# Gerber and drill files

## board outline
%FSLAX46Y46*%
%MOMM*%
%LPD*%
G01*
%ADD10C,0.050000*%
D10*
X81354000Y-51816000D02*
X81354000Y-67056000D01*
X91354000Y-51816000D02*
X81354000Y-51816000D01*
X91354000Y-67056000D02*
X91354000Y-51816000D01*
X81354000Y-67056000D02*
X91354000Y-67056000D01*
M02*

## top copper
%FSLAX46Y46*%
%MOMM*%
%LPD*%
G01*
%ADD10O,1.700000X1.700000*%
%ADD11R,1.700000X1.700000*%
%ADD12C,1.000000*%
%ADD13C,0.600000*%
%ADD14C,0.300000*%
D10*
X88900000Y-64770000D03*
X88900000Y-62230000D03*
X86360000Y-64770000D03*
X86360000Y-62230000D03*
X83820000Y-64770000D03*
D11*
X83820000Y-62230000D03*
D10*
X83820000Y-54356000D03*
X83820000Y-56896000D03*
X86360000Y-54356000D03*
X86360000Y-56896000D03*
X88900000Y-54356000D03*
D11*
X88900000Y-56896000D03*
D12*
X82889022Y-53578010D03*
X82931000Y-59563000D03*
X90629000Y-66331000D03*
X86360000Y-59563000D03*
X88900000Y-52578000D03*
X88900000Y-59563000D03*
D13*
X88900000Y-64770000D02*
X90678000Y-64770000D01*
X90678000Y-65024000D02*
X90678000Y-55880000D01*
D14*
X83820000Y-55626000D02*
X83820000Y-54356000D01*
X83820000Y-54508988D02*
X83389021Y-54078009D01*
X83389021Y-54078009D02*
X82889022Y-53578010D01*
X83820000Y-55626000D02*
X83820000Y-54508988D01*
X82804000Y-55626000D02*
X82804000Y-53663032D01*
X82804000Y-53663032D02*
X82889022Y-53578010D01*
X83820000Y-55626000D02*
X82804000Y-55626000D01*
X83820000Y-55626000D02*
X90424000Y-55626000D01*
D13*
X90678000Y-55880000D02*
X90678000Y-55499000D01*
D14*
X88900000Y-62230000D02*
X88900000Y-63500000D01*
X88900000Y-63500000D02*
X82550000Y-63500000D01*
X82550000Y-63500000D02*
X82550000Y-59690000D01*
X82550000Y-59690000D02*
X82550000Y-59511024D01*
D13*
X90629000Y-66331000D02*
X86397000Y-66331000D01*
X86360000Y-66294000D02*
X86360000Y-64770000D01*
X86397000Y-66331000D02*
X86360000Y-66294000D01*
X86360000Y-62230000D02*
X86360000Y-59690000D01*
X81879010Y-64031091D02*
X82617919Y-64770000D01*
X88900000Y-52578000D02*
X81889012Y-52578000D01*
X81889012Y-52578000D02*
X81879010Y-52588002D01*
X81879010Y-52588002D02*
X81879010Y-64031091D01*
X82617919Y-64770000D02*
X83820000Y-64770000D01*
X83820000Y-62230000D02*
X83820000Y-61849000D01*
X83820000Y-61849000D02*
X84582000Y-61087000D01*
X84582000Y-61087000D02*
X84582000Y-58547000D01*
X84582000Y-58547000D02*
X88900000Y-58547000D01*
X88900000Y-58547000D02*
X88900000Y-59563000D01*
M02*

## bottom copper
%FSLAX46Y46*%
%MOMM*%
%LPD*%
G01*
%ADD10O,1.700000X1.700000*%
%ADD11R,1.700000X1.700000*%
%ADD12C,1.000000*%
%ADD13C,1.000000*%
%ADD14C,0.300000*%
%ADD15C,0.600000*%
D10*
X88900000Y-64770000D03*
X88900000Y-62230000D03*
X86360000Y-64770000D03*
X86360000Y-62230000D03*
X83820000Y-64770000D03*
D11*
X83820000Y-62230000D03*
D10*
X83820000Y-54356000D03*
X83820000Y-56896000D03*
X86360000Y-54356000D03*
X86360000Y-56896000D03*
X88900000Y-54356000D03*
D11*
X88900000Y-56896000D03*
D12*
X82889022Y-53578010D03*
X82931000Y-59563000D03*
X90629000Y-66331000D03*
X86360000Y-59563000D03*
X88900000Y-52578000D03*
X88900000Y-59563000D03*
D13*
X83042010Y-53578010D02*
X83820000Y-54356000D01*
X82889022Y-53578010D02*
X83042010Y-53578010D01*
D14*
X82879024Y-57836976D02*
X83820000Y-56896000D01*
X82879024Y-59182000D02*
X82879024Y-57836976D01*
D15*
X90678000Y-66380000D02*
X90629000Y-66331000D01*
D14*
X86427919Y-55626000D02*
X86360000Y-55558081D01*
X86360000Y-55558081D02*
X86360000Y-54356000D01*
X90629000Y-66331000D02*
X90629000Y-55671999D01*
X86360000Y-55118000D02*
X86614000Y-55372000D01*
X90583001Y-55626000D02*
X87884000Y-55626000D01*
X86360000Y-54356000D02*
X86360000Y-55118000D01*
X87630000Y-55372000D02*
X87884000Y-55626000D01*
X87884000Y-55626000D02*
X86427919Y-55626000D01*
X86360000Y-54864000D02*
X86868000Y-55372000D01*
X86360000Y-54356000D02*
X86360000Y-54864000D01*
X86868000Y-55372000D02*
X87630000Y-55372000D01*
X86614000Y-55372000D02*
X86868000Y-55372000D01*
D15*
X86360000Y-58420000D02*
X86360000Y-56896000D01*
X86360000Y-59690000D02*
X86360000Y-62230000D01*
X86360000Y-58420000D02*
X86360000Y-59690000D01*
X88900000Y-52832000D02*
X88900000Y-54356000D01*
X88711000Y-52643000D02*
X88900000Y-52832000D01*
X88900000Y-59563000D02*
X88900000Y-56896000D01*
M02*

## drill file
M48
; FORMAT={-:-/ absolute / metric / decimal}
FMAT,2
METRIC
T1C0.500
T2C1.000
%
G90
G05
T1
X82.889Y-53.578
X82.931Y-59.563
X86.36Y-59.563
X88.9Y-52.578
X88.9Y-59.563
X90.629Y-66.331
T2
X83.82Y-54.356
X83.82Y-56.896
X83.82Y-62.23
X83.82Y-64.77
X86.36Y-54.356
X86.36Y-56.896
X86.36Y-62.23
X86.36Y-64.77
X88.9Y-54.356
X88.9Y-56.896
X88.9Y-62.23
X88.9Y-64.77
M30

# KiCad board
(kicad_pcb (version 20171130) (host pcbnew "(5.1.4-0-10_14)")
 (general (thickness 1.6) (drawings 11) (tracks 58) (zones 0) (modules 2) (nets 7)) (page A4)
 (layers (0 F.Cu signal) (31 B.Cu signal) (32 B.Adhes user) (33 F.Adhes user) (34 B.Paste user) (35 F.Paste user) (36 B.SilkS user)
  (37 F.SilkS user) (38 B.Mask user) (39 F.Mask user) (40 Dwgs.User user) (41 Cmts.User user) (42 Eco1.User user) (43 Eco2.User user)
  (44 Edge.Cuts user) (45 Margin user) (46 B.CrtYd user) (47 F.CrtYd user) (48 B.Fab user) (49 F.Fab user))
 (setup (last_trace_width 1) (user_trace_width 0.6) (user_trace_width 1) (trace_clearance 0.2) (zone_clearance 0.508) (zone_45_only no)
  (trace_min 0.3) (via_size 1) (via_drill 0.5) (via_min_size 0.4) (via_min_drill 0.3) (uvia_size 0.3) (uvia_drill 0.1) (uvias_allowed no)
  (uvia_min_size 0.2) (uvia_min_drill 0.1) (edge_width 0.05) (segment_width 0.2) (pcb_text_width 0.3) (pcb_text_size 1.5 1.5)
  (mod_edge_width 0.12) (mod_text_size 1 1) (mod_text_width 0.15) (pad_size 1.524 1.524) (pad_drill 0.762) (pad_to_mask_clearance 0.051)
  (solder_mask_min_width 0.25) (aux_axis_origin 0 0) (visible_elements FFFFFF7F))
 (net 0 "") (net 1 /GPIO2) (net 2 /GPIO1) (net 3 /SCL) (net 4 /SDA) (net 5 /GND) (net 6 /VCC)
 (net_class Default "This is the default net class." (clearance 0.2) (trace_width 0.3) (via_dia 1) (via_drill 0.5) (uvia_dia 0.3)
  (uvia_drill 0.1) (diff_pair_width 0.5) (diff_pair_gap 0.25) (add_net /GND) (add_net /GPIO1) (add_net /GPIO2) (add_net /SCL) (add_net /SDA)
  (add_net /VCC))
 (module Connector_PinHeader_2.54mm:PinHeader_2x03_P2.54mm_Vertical (layer B.Cu) (at 83.82 62.23 270)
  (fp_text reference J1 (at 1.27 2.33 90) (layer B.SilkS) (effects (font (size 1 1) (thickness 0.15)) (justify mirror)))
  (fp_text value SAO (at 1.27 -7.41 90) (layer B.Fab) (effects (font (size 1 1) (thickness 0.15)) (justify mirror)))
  (pad 6 thru_hole oval (at 2.54 -5.08 270) (size 1.7 1.7) (drill 1) (layers *.Cu *.Mask) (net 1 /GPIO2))
  (pad 5 thru_hole oval (at 0 -5.08 270) (size 1.7 1.7) (drill 1) (layers *.Cu *.Mask) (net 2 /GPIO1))
  (pad 4 thru_hole oval (at 2.54 -2.54 270) (size 1.7 1.7) (drill 1) (layers *.Cu *.Mask) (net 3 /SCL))
  (pad 3 thru_hole oval (at 0 -2.54 270) (size 1.7 1.7) (drill 1) (layers *.Cu *.Mask) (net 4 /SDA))
  (pad 2 thru_hole oval (at 2.54 0 270) (size 1.7 1.7) (drill 1) (layers *.Cu *.Mask) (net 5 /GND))
  (pad 1 thru_hole rect (at 0 0 270) (size 1.7 1.7) (drill 1) (layers *.Cu *.Mask) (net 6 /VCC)))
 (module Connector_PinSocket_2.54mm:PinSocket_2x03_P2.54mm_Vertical (layer F.Cu) (at 88.9 56.896 270)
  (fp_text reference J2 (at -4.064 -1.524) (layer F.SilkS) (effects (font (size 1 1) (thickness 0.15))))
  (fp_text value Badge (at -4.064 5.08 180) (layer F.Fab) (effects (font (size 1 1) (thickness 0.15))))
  (pad 6 thru_hole oval (at -2.54 5.08 270) (size 1.7 1.7) (drill 1) (layers *.Cu *.Mask) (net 1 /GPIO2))
  (pad 5 thru_hole oval (at 0 5.08 270) (size 1.7 1.7) (drill 1) (layers *.Cu *.Mask) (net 2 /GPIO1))
  (pad 4 thru_hole oval (at -2.54 2.54 270) (size 1.7 1.7) (drill 1) (layers *.Cu *.Mask) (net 3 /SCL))
  (pad 3 thru_hole oval (at 0 2.54 270) (size 1.7 1.7) (drill 1) (layers *.Cu *.Mask) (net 4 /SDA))
  (pad 2 thru_hole oval (at -2.54 0 270) (size 1.7 1.7) (drill 1) (layers *.Cu *.Mask) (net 5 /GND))
  (pad 1 thru_hole rect (at 0 0 270) (size 1.7 1.7) (drill 1) (layers *.Cu *.Mask) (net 6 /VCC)))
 (gr_line (start 81.354 51.816) (end 81.354 67.056) (layer Edge.Cuts) (width 0.05))
 (gr_line (start 91.354 51.816) (end 81.354 51.816) (layer Edge.Cuts) (width 0.05))
 (gr_line (start 91.354 67.056) (end 91.354 51.816) (layer Edge.Cuts) (width 0.05))
 (gr_line (start 81.354 67.056) (end 91.354 67.056) (layer Edge.Cuts) (width 0.05))
 (segment (start 88.9 64.77) (end 90.678 64.77) (width 0.6) (layer F.Cu) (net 1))
 (segment (start 90.678 65.024) (end 90.678 55.88) (width 0.6) (layer F.Cu) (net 1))
 (segment (start 83.82 55.626) (end 83.82 54.356) (width 0.3) (layer F.Cu) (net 1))
 (via (at 82.889022 53.57801) (size 1) (drill 0.5) (layers F.Cu B.Cu) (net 1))
 (segment (start 83.82 54.508988) (end 83.389021 54.078009) (width 0.3) (layer F.Cu) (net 1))
 (segment (start 83.389021 54.078009) (end 82.889022 53.57801) (width 0.3) (layer F.Cu) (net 1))
 (segment (start 83.82 55.626) (end 83.82 54.508988) (width 0.3) (layer F.Cu) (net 1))
 (segment (start 82.804 55.626) (end 82.804 53.663032) (width 0.3) (layer F.Cu) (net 1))
 (segment (start 82.804 53.663032) (end 82.889022 53.57801) (width 0.3) (layer F.Cu) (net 1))
 (segment (start 83.82 55.626) (end 82.804 55.626) (width 0.3) (layer F.Cu) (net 1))
 (segment (start 83.82 55.626) (end 90.424 55.626) (width 0.3) (layer F.Cu) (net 1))
 (segment (start 90.678 55.88) (end 90.678 55.499) (width 0.6) (layer F.Cu) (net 1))
 (segment (start 83.04201 53.57801) (end 83.82 54.356) (width 1) (layer B.Cu) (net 1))
 (segment (start 82.889022 53.57801) (end 83.04201 53.57801) (width 1) (layer B.Cu) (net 1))
 (segment (start 88.9 62.23) (end 88.9 63.5) (width 0.3) (layer F.Cu) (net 2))
 (segment (start 88.9 63.5) (end 82.55 63.5) (width 0.3) (layer F.Cu) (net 2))
 (segment (start 82.55 63.5) (end 82.55 59.69) (width 0.3) (layer F.Cu) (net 2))
 (via (at 82.931 59.563) (size 1) (drill 0.5) (layers F.Cu B.Cu) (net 2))
 (segment (start 82.55 59.69) (end 82.55 59.511024) (width 0.3) (layer F.Cu) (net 2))
 (segment (start 82.879024 57.836976) (end 83.82 56.896) (width 0.3) (layer B.Cu) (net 2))
 (segment (start 82.879024 59.182) (end 82.879024 57.836976) (width 0.3) (layer B.Cu) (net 2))
 (segment (start 90.678 66.38) (end 90.629 66.331) (width 0.6) (layer B.Cu) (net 3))
 (via (at 90.629 66.331) (size 1) (drill 0.5) (layers F.Cu B.Cu) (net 3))
 (segment (start 90.629 66.331) (end 86.397 66.331) (width 0.6) (layer F.Cu) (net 3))
 (segment (start 86.36 66.294) (end 86.36 64.77) (width 0.6) (layer F.Cu) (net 3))
 (segment (start 86.397 66.331) (end 86.36 66.294) (width 0.6) (layer F.Cu) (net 3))
 (segment (start 86.427919 55.626) (end 86.36 55.558081) (width 0.3) (layer B.Cu) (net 3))
 (segment (start 86.36 55.558081) (end 86.36 54.356) (width 0.3) (layer B.Cu) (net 3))
 (segment (start 90.629 66.331) (end 90.629 55.671999) (width 0.3) (layer B.Cu) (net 3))
 (segment (start 86.36 55.118) (end 86.614 55.372) (width 0.3) (layer B.Cu) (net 3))
 (segment (start 90.583001 55.626) (end 87.884 55.626) (width 0.3) (layer B.Cu) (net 3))
 (segment (start 86.36 54.356) (end 86.36 55.118) (width 0.3) (layer B.Cu) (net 3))
 (segment (start 87.63 55.372) (end 87.884 55.626) (width 0.3) (layer B.Cu) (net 3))
 (segment (start 87.884 55.626) (end 86.427919 55.626) (width 0.3) (layer B.Cu) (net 3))
 (segment (start 86.36 54.864) (end 86.868 55.372) (width 0.3) (layer B.Cu) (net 3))
 (segment (start 86.36 54.356) (end 86.36 54.864) (width 0.3) (layer B.Cu) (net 3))
 (segment (start 86.868 55.372) (end 87.63 55.372) (width 0.3) (layer B.Cu) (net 3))
 (segment (start 86.614 55.372) (end 86.868 55.372) (width 0.3) (layer B.Cu) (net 3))
 (segment (start 86.36 58.42) (end 86.36 56.896) (width 0.6) (layer B.Cu) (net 4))
 (via (at 86.36 59.563) (size 1) (drill 0.5) (layers F.Cu B.Cu) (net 4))
 (segment (start 86.36 62.23) (end 86.36 59.69) (width 0.6) (layer F.Cu) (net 4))
 (segment (start 86.36 59.69) (end 86.36 62.23) (width 0.6) (layer B.Cu) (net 4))
 (segment (start 86.36 58.42) (end 86.36 59.69) (width 0.6) (layer B.Cu) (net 4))
 (via (at 88.9 52.578) (size 1) (drill 0.5) (layers F.Cu B.Cu) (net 5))
 (segment (start 88.9 52.832) (end 88.9 54.356) (width 0.6) (layer B.Cu) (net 5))
 (segment (start 88.711 52.643) (end 88.9 52.832) (width 0.6) (layer B.Cu) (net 5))
 (segment (start 81.87901 64.031091) (end 82.617919 64.77) (width 0.6) (layer F.Cu) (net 5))
 (segment (start 88.9 52.578) (end 81.889012 52.578) (width 0.6) (layer F.Cu) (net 5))
 (segment (start 81.889012 52.578) (end 81.87901 52.588002) (width 0.6) (layer F.Cu) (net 5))
 (segment (start 81.87901 52.588002) (end 81.87901 64.031091) (width 0.6) (layer F.Cu) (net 5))
 (segment (start 82.617919 64.77) (end 83.82 64.77) (width 0.6) (layer F.Cu) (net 5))
 (segment (start 83.82 62.23) (end 83.82 61.849) (width 0.6) (layer F.Cu) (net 6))
 (segment (start 83.82 61.849) (end 84.582 61.087) (width 0.6) (layer F.Cu) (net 6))
 (segment (start 84.582 61.087) (end 84.582 58.547) (width 0.6) (layer F.Cu) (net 6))
 (segment (start 84.582 58.547) (end 88.9 58.547) (width 0.6) (layer F.Cu) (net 6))
 (via (at 88.9 59.563) (size 1) (drill 0.5) (layers F.Cu B.Cu) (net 6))
 (segment (start 88.9 58.547) (end 88.9 59.563) (width 0.6) (layer F.Cu) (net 6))
 (segment (start 88.9 59.563) (end 88.9 56.896) (width 0.6) (layer B.Cu) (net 6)))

